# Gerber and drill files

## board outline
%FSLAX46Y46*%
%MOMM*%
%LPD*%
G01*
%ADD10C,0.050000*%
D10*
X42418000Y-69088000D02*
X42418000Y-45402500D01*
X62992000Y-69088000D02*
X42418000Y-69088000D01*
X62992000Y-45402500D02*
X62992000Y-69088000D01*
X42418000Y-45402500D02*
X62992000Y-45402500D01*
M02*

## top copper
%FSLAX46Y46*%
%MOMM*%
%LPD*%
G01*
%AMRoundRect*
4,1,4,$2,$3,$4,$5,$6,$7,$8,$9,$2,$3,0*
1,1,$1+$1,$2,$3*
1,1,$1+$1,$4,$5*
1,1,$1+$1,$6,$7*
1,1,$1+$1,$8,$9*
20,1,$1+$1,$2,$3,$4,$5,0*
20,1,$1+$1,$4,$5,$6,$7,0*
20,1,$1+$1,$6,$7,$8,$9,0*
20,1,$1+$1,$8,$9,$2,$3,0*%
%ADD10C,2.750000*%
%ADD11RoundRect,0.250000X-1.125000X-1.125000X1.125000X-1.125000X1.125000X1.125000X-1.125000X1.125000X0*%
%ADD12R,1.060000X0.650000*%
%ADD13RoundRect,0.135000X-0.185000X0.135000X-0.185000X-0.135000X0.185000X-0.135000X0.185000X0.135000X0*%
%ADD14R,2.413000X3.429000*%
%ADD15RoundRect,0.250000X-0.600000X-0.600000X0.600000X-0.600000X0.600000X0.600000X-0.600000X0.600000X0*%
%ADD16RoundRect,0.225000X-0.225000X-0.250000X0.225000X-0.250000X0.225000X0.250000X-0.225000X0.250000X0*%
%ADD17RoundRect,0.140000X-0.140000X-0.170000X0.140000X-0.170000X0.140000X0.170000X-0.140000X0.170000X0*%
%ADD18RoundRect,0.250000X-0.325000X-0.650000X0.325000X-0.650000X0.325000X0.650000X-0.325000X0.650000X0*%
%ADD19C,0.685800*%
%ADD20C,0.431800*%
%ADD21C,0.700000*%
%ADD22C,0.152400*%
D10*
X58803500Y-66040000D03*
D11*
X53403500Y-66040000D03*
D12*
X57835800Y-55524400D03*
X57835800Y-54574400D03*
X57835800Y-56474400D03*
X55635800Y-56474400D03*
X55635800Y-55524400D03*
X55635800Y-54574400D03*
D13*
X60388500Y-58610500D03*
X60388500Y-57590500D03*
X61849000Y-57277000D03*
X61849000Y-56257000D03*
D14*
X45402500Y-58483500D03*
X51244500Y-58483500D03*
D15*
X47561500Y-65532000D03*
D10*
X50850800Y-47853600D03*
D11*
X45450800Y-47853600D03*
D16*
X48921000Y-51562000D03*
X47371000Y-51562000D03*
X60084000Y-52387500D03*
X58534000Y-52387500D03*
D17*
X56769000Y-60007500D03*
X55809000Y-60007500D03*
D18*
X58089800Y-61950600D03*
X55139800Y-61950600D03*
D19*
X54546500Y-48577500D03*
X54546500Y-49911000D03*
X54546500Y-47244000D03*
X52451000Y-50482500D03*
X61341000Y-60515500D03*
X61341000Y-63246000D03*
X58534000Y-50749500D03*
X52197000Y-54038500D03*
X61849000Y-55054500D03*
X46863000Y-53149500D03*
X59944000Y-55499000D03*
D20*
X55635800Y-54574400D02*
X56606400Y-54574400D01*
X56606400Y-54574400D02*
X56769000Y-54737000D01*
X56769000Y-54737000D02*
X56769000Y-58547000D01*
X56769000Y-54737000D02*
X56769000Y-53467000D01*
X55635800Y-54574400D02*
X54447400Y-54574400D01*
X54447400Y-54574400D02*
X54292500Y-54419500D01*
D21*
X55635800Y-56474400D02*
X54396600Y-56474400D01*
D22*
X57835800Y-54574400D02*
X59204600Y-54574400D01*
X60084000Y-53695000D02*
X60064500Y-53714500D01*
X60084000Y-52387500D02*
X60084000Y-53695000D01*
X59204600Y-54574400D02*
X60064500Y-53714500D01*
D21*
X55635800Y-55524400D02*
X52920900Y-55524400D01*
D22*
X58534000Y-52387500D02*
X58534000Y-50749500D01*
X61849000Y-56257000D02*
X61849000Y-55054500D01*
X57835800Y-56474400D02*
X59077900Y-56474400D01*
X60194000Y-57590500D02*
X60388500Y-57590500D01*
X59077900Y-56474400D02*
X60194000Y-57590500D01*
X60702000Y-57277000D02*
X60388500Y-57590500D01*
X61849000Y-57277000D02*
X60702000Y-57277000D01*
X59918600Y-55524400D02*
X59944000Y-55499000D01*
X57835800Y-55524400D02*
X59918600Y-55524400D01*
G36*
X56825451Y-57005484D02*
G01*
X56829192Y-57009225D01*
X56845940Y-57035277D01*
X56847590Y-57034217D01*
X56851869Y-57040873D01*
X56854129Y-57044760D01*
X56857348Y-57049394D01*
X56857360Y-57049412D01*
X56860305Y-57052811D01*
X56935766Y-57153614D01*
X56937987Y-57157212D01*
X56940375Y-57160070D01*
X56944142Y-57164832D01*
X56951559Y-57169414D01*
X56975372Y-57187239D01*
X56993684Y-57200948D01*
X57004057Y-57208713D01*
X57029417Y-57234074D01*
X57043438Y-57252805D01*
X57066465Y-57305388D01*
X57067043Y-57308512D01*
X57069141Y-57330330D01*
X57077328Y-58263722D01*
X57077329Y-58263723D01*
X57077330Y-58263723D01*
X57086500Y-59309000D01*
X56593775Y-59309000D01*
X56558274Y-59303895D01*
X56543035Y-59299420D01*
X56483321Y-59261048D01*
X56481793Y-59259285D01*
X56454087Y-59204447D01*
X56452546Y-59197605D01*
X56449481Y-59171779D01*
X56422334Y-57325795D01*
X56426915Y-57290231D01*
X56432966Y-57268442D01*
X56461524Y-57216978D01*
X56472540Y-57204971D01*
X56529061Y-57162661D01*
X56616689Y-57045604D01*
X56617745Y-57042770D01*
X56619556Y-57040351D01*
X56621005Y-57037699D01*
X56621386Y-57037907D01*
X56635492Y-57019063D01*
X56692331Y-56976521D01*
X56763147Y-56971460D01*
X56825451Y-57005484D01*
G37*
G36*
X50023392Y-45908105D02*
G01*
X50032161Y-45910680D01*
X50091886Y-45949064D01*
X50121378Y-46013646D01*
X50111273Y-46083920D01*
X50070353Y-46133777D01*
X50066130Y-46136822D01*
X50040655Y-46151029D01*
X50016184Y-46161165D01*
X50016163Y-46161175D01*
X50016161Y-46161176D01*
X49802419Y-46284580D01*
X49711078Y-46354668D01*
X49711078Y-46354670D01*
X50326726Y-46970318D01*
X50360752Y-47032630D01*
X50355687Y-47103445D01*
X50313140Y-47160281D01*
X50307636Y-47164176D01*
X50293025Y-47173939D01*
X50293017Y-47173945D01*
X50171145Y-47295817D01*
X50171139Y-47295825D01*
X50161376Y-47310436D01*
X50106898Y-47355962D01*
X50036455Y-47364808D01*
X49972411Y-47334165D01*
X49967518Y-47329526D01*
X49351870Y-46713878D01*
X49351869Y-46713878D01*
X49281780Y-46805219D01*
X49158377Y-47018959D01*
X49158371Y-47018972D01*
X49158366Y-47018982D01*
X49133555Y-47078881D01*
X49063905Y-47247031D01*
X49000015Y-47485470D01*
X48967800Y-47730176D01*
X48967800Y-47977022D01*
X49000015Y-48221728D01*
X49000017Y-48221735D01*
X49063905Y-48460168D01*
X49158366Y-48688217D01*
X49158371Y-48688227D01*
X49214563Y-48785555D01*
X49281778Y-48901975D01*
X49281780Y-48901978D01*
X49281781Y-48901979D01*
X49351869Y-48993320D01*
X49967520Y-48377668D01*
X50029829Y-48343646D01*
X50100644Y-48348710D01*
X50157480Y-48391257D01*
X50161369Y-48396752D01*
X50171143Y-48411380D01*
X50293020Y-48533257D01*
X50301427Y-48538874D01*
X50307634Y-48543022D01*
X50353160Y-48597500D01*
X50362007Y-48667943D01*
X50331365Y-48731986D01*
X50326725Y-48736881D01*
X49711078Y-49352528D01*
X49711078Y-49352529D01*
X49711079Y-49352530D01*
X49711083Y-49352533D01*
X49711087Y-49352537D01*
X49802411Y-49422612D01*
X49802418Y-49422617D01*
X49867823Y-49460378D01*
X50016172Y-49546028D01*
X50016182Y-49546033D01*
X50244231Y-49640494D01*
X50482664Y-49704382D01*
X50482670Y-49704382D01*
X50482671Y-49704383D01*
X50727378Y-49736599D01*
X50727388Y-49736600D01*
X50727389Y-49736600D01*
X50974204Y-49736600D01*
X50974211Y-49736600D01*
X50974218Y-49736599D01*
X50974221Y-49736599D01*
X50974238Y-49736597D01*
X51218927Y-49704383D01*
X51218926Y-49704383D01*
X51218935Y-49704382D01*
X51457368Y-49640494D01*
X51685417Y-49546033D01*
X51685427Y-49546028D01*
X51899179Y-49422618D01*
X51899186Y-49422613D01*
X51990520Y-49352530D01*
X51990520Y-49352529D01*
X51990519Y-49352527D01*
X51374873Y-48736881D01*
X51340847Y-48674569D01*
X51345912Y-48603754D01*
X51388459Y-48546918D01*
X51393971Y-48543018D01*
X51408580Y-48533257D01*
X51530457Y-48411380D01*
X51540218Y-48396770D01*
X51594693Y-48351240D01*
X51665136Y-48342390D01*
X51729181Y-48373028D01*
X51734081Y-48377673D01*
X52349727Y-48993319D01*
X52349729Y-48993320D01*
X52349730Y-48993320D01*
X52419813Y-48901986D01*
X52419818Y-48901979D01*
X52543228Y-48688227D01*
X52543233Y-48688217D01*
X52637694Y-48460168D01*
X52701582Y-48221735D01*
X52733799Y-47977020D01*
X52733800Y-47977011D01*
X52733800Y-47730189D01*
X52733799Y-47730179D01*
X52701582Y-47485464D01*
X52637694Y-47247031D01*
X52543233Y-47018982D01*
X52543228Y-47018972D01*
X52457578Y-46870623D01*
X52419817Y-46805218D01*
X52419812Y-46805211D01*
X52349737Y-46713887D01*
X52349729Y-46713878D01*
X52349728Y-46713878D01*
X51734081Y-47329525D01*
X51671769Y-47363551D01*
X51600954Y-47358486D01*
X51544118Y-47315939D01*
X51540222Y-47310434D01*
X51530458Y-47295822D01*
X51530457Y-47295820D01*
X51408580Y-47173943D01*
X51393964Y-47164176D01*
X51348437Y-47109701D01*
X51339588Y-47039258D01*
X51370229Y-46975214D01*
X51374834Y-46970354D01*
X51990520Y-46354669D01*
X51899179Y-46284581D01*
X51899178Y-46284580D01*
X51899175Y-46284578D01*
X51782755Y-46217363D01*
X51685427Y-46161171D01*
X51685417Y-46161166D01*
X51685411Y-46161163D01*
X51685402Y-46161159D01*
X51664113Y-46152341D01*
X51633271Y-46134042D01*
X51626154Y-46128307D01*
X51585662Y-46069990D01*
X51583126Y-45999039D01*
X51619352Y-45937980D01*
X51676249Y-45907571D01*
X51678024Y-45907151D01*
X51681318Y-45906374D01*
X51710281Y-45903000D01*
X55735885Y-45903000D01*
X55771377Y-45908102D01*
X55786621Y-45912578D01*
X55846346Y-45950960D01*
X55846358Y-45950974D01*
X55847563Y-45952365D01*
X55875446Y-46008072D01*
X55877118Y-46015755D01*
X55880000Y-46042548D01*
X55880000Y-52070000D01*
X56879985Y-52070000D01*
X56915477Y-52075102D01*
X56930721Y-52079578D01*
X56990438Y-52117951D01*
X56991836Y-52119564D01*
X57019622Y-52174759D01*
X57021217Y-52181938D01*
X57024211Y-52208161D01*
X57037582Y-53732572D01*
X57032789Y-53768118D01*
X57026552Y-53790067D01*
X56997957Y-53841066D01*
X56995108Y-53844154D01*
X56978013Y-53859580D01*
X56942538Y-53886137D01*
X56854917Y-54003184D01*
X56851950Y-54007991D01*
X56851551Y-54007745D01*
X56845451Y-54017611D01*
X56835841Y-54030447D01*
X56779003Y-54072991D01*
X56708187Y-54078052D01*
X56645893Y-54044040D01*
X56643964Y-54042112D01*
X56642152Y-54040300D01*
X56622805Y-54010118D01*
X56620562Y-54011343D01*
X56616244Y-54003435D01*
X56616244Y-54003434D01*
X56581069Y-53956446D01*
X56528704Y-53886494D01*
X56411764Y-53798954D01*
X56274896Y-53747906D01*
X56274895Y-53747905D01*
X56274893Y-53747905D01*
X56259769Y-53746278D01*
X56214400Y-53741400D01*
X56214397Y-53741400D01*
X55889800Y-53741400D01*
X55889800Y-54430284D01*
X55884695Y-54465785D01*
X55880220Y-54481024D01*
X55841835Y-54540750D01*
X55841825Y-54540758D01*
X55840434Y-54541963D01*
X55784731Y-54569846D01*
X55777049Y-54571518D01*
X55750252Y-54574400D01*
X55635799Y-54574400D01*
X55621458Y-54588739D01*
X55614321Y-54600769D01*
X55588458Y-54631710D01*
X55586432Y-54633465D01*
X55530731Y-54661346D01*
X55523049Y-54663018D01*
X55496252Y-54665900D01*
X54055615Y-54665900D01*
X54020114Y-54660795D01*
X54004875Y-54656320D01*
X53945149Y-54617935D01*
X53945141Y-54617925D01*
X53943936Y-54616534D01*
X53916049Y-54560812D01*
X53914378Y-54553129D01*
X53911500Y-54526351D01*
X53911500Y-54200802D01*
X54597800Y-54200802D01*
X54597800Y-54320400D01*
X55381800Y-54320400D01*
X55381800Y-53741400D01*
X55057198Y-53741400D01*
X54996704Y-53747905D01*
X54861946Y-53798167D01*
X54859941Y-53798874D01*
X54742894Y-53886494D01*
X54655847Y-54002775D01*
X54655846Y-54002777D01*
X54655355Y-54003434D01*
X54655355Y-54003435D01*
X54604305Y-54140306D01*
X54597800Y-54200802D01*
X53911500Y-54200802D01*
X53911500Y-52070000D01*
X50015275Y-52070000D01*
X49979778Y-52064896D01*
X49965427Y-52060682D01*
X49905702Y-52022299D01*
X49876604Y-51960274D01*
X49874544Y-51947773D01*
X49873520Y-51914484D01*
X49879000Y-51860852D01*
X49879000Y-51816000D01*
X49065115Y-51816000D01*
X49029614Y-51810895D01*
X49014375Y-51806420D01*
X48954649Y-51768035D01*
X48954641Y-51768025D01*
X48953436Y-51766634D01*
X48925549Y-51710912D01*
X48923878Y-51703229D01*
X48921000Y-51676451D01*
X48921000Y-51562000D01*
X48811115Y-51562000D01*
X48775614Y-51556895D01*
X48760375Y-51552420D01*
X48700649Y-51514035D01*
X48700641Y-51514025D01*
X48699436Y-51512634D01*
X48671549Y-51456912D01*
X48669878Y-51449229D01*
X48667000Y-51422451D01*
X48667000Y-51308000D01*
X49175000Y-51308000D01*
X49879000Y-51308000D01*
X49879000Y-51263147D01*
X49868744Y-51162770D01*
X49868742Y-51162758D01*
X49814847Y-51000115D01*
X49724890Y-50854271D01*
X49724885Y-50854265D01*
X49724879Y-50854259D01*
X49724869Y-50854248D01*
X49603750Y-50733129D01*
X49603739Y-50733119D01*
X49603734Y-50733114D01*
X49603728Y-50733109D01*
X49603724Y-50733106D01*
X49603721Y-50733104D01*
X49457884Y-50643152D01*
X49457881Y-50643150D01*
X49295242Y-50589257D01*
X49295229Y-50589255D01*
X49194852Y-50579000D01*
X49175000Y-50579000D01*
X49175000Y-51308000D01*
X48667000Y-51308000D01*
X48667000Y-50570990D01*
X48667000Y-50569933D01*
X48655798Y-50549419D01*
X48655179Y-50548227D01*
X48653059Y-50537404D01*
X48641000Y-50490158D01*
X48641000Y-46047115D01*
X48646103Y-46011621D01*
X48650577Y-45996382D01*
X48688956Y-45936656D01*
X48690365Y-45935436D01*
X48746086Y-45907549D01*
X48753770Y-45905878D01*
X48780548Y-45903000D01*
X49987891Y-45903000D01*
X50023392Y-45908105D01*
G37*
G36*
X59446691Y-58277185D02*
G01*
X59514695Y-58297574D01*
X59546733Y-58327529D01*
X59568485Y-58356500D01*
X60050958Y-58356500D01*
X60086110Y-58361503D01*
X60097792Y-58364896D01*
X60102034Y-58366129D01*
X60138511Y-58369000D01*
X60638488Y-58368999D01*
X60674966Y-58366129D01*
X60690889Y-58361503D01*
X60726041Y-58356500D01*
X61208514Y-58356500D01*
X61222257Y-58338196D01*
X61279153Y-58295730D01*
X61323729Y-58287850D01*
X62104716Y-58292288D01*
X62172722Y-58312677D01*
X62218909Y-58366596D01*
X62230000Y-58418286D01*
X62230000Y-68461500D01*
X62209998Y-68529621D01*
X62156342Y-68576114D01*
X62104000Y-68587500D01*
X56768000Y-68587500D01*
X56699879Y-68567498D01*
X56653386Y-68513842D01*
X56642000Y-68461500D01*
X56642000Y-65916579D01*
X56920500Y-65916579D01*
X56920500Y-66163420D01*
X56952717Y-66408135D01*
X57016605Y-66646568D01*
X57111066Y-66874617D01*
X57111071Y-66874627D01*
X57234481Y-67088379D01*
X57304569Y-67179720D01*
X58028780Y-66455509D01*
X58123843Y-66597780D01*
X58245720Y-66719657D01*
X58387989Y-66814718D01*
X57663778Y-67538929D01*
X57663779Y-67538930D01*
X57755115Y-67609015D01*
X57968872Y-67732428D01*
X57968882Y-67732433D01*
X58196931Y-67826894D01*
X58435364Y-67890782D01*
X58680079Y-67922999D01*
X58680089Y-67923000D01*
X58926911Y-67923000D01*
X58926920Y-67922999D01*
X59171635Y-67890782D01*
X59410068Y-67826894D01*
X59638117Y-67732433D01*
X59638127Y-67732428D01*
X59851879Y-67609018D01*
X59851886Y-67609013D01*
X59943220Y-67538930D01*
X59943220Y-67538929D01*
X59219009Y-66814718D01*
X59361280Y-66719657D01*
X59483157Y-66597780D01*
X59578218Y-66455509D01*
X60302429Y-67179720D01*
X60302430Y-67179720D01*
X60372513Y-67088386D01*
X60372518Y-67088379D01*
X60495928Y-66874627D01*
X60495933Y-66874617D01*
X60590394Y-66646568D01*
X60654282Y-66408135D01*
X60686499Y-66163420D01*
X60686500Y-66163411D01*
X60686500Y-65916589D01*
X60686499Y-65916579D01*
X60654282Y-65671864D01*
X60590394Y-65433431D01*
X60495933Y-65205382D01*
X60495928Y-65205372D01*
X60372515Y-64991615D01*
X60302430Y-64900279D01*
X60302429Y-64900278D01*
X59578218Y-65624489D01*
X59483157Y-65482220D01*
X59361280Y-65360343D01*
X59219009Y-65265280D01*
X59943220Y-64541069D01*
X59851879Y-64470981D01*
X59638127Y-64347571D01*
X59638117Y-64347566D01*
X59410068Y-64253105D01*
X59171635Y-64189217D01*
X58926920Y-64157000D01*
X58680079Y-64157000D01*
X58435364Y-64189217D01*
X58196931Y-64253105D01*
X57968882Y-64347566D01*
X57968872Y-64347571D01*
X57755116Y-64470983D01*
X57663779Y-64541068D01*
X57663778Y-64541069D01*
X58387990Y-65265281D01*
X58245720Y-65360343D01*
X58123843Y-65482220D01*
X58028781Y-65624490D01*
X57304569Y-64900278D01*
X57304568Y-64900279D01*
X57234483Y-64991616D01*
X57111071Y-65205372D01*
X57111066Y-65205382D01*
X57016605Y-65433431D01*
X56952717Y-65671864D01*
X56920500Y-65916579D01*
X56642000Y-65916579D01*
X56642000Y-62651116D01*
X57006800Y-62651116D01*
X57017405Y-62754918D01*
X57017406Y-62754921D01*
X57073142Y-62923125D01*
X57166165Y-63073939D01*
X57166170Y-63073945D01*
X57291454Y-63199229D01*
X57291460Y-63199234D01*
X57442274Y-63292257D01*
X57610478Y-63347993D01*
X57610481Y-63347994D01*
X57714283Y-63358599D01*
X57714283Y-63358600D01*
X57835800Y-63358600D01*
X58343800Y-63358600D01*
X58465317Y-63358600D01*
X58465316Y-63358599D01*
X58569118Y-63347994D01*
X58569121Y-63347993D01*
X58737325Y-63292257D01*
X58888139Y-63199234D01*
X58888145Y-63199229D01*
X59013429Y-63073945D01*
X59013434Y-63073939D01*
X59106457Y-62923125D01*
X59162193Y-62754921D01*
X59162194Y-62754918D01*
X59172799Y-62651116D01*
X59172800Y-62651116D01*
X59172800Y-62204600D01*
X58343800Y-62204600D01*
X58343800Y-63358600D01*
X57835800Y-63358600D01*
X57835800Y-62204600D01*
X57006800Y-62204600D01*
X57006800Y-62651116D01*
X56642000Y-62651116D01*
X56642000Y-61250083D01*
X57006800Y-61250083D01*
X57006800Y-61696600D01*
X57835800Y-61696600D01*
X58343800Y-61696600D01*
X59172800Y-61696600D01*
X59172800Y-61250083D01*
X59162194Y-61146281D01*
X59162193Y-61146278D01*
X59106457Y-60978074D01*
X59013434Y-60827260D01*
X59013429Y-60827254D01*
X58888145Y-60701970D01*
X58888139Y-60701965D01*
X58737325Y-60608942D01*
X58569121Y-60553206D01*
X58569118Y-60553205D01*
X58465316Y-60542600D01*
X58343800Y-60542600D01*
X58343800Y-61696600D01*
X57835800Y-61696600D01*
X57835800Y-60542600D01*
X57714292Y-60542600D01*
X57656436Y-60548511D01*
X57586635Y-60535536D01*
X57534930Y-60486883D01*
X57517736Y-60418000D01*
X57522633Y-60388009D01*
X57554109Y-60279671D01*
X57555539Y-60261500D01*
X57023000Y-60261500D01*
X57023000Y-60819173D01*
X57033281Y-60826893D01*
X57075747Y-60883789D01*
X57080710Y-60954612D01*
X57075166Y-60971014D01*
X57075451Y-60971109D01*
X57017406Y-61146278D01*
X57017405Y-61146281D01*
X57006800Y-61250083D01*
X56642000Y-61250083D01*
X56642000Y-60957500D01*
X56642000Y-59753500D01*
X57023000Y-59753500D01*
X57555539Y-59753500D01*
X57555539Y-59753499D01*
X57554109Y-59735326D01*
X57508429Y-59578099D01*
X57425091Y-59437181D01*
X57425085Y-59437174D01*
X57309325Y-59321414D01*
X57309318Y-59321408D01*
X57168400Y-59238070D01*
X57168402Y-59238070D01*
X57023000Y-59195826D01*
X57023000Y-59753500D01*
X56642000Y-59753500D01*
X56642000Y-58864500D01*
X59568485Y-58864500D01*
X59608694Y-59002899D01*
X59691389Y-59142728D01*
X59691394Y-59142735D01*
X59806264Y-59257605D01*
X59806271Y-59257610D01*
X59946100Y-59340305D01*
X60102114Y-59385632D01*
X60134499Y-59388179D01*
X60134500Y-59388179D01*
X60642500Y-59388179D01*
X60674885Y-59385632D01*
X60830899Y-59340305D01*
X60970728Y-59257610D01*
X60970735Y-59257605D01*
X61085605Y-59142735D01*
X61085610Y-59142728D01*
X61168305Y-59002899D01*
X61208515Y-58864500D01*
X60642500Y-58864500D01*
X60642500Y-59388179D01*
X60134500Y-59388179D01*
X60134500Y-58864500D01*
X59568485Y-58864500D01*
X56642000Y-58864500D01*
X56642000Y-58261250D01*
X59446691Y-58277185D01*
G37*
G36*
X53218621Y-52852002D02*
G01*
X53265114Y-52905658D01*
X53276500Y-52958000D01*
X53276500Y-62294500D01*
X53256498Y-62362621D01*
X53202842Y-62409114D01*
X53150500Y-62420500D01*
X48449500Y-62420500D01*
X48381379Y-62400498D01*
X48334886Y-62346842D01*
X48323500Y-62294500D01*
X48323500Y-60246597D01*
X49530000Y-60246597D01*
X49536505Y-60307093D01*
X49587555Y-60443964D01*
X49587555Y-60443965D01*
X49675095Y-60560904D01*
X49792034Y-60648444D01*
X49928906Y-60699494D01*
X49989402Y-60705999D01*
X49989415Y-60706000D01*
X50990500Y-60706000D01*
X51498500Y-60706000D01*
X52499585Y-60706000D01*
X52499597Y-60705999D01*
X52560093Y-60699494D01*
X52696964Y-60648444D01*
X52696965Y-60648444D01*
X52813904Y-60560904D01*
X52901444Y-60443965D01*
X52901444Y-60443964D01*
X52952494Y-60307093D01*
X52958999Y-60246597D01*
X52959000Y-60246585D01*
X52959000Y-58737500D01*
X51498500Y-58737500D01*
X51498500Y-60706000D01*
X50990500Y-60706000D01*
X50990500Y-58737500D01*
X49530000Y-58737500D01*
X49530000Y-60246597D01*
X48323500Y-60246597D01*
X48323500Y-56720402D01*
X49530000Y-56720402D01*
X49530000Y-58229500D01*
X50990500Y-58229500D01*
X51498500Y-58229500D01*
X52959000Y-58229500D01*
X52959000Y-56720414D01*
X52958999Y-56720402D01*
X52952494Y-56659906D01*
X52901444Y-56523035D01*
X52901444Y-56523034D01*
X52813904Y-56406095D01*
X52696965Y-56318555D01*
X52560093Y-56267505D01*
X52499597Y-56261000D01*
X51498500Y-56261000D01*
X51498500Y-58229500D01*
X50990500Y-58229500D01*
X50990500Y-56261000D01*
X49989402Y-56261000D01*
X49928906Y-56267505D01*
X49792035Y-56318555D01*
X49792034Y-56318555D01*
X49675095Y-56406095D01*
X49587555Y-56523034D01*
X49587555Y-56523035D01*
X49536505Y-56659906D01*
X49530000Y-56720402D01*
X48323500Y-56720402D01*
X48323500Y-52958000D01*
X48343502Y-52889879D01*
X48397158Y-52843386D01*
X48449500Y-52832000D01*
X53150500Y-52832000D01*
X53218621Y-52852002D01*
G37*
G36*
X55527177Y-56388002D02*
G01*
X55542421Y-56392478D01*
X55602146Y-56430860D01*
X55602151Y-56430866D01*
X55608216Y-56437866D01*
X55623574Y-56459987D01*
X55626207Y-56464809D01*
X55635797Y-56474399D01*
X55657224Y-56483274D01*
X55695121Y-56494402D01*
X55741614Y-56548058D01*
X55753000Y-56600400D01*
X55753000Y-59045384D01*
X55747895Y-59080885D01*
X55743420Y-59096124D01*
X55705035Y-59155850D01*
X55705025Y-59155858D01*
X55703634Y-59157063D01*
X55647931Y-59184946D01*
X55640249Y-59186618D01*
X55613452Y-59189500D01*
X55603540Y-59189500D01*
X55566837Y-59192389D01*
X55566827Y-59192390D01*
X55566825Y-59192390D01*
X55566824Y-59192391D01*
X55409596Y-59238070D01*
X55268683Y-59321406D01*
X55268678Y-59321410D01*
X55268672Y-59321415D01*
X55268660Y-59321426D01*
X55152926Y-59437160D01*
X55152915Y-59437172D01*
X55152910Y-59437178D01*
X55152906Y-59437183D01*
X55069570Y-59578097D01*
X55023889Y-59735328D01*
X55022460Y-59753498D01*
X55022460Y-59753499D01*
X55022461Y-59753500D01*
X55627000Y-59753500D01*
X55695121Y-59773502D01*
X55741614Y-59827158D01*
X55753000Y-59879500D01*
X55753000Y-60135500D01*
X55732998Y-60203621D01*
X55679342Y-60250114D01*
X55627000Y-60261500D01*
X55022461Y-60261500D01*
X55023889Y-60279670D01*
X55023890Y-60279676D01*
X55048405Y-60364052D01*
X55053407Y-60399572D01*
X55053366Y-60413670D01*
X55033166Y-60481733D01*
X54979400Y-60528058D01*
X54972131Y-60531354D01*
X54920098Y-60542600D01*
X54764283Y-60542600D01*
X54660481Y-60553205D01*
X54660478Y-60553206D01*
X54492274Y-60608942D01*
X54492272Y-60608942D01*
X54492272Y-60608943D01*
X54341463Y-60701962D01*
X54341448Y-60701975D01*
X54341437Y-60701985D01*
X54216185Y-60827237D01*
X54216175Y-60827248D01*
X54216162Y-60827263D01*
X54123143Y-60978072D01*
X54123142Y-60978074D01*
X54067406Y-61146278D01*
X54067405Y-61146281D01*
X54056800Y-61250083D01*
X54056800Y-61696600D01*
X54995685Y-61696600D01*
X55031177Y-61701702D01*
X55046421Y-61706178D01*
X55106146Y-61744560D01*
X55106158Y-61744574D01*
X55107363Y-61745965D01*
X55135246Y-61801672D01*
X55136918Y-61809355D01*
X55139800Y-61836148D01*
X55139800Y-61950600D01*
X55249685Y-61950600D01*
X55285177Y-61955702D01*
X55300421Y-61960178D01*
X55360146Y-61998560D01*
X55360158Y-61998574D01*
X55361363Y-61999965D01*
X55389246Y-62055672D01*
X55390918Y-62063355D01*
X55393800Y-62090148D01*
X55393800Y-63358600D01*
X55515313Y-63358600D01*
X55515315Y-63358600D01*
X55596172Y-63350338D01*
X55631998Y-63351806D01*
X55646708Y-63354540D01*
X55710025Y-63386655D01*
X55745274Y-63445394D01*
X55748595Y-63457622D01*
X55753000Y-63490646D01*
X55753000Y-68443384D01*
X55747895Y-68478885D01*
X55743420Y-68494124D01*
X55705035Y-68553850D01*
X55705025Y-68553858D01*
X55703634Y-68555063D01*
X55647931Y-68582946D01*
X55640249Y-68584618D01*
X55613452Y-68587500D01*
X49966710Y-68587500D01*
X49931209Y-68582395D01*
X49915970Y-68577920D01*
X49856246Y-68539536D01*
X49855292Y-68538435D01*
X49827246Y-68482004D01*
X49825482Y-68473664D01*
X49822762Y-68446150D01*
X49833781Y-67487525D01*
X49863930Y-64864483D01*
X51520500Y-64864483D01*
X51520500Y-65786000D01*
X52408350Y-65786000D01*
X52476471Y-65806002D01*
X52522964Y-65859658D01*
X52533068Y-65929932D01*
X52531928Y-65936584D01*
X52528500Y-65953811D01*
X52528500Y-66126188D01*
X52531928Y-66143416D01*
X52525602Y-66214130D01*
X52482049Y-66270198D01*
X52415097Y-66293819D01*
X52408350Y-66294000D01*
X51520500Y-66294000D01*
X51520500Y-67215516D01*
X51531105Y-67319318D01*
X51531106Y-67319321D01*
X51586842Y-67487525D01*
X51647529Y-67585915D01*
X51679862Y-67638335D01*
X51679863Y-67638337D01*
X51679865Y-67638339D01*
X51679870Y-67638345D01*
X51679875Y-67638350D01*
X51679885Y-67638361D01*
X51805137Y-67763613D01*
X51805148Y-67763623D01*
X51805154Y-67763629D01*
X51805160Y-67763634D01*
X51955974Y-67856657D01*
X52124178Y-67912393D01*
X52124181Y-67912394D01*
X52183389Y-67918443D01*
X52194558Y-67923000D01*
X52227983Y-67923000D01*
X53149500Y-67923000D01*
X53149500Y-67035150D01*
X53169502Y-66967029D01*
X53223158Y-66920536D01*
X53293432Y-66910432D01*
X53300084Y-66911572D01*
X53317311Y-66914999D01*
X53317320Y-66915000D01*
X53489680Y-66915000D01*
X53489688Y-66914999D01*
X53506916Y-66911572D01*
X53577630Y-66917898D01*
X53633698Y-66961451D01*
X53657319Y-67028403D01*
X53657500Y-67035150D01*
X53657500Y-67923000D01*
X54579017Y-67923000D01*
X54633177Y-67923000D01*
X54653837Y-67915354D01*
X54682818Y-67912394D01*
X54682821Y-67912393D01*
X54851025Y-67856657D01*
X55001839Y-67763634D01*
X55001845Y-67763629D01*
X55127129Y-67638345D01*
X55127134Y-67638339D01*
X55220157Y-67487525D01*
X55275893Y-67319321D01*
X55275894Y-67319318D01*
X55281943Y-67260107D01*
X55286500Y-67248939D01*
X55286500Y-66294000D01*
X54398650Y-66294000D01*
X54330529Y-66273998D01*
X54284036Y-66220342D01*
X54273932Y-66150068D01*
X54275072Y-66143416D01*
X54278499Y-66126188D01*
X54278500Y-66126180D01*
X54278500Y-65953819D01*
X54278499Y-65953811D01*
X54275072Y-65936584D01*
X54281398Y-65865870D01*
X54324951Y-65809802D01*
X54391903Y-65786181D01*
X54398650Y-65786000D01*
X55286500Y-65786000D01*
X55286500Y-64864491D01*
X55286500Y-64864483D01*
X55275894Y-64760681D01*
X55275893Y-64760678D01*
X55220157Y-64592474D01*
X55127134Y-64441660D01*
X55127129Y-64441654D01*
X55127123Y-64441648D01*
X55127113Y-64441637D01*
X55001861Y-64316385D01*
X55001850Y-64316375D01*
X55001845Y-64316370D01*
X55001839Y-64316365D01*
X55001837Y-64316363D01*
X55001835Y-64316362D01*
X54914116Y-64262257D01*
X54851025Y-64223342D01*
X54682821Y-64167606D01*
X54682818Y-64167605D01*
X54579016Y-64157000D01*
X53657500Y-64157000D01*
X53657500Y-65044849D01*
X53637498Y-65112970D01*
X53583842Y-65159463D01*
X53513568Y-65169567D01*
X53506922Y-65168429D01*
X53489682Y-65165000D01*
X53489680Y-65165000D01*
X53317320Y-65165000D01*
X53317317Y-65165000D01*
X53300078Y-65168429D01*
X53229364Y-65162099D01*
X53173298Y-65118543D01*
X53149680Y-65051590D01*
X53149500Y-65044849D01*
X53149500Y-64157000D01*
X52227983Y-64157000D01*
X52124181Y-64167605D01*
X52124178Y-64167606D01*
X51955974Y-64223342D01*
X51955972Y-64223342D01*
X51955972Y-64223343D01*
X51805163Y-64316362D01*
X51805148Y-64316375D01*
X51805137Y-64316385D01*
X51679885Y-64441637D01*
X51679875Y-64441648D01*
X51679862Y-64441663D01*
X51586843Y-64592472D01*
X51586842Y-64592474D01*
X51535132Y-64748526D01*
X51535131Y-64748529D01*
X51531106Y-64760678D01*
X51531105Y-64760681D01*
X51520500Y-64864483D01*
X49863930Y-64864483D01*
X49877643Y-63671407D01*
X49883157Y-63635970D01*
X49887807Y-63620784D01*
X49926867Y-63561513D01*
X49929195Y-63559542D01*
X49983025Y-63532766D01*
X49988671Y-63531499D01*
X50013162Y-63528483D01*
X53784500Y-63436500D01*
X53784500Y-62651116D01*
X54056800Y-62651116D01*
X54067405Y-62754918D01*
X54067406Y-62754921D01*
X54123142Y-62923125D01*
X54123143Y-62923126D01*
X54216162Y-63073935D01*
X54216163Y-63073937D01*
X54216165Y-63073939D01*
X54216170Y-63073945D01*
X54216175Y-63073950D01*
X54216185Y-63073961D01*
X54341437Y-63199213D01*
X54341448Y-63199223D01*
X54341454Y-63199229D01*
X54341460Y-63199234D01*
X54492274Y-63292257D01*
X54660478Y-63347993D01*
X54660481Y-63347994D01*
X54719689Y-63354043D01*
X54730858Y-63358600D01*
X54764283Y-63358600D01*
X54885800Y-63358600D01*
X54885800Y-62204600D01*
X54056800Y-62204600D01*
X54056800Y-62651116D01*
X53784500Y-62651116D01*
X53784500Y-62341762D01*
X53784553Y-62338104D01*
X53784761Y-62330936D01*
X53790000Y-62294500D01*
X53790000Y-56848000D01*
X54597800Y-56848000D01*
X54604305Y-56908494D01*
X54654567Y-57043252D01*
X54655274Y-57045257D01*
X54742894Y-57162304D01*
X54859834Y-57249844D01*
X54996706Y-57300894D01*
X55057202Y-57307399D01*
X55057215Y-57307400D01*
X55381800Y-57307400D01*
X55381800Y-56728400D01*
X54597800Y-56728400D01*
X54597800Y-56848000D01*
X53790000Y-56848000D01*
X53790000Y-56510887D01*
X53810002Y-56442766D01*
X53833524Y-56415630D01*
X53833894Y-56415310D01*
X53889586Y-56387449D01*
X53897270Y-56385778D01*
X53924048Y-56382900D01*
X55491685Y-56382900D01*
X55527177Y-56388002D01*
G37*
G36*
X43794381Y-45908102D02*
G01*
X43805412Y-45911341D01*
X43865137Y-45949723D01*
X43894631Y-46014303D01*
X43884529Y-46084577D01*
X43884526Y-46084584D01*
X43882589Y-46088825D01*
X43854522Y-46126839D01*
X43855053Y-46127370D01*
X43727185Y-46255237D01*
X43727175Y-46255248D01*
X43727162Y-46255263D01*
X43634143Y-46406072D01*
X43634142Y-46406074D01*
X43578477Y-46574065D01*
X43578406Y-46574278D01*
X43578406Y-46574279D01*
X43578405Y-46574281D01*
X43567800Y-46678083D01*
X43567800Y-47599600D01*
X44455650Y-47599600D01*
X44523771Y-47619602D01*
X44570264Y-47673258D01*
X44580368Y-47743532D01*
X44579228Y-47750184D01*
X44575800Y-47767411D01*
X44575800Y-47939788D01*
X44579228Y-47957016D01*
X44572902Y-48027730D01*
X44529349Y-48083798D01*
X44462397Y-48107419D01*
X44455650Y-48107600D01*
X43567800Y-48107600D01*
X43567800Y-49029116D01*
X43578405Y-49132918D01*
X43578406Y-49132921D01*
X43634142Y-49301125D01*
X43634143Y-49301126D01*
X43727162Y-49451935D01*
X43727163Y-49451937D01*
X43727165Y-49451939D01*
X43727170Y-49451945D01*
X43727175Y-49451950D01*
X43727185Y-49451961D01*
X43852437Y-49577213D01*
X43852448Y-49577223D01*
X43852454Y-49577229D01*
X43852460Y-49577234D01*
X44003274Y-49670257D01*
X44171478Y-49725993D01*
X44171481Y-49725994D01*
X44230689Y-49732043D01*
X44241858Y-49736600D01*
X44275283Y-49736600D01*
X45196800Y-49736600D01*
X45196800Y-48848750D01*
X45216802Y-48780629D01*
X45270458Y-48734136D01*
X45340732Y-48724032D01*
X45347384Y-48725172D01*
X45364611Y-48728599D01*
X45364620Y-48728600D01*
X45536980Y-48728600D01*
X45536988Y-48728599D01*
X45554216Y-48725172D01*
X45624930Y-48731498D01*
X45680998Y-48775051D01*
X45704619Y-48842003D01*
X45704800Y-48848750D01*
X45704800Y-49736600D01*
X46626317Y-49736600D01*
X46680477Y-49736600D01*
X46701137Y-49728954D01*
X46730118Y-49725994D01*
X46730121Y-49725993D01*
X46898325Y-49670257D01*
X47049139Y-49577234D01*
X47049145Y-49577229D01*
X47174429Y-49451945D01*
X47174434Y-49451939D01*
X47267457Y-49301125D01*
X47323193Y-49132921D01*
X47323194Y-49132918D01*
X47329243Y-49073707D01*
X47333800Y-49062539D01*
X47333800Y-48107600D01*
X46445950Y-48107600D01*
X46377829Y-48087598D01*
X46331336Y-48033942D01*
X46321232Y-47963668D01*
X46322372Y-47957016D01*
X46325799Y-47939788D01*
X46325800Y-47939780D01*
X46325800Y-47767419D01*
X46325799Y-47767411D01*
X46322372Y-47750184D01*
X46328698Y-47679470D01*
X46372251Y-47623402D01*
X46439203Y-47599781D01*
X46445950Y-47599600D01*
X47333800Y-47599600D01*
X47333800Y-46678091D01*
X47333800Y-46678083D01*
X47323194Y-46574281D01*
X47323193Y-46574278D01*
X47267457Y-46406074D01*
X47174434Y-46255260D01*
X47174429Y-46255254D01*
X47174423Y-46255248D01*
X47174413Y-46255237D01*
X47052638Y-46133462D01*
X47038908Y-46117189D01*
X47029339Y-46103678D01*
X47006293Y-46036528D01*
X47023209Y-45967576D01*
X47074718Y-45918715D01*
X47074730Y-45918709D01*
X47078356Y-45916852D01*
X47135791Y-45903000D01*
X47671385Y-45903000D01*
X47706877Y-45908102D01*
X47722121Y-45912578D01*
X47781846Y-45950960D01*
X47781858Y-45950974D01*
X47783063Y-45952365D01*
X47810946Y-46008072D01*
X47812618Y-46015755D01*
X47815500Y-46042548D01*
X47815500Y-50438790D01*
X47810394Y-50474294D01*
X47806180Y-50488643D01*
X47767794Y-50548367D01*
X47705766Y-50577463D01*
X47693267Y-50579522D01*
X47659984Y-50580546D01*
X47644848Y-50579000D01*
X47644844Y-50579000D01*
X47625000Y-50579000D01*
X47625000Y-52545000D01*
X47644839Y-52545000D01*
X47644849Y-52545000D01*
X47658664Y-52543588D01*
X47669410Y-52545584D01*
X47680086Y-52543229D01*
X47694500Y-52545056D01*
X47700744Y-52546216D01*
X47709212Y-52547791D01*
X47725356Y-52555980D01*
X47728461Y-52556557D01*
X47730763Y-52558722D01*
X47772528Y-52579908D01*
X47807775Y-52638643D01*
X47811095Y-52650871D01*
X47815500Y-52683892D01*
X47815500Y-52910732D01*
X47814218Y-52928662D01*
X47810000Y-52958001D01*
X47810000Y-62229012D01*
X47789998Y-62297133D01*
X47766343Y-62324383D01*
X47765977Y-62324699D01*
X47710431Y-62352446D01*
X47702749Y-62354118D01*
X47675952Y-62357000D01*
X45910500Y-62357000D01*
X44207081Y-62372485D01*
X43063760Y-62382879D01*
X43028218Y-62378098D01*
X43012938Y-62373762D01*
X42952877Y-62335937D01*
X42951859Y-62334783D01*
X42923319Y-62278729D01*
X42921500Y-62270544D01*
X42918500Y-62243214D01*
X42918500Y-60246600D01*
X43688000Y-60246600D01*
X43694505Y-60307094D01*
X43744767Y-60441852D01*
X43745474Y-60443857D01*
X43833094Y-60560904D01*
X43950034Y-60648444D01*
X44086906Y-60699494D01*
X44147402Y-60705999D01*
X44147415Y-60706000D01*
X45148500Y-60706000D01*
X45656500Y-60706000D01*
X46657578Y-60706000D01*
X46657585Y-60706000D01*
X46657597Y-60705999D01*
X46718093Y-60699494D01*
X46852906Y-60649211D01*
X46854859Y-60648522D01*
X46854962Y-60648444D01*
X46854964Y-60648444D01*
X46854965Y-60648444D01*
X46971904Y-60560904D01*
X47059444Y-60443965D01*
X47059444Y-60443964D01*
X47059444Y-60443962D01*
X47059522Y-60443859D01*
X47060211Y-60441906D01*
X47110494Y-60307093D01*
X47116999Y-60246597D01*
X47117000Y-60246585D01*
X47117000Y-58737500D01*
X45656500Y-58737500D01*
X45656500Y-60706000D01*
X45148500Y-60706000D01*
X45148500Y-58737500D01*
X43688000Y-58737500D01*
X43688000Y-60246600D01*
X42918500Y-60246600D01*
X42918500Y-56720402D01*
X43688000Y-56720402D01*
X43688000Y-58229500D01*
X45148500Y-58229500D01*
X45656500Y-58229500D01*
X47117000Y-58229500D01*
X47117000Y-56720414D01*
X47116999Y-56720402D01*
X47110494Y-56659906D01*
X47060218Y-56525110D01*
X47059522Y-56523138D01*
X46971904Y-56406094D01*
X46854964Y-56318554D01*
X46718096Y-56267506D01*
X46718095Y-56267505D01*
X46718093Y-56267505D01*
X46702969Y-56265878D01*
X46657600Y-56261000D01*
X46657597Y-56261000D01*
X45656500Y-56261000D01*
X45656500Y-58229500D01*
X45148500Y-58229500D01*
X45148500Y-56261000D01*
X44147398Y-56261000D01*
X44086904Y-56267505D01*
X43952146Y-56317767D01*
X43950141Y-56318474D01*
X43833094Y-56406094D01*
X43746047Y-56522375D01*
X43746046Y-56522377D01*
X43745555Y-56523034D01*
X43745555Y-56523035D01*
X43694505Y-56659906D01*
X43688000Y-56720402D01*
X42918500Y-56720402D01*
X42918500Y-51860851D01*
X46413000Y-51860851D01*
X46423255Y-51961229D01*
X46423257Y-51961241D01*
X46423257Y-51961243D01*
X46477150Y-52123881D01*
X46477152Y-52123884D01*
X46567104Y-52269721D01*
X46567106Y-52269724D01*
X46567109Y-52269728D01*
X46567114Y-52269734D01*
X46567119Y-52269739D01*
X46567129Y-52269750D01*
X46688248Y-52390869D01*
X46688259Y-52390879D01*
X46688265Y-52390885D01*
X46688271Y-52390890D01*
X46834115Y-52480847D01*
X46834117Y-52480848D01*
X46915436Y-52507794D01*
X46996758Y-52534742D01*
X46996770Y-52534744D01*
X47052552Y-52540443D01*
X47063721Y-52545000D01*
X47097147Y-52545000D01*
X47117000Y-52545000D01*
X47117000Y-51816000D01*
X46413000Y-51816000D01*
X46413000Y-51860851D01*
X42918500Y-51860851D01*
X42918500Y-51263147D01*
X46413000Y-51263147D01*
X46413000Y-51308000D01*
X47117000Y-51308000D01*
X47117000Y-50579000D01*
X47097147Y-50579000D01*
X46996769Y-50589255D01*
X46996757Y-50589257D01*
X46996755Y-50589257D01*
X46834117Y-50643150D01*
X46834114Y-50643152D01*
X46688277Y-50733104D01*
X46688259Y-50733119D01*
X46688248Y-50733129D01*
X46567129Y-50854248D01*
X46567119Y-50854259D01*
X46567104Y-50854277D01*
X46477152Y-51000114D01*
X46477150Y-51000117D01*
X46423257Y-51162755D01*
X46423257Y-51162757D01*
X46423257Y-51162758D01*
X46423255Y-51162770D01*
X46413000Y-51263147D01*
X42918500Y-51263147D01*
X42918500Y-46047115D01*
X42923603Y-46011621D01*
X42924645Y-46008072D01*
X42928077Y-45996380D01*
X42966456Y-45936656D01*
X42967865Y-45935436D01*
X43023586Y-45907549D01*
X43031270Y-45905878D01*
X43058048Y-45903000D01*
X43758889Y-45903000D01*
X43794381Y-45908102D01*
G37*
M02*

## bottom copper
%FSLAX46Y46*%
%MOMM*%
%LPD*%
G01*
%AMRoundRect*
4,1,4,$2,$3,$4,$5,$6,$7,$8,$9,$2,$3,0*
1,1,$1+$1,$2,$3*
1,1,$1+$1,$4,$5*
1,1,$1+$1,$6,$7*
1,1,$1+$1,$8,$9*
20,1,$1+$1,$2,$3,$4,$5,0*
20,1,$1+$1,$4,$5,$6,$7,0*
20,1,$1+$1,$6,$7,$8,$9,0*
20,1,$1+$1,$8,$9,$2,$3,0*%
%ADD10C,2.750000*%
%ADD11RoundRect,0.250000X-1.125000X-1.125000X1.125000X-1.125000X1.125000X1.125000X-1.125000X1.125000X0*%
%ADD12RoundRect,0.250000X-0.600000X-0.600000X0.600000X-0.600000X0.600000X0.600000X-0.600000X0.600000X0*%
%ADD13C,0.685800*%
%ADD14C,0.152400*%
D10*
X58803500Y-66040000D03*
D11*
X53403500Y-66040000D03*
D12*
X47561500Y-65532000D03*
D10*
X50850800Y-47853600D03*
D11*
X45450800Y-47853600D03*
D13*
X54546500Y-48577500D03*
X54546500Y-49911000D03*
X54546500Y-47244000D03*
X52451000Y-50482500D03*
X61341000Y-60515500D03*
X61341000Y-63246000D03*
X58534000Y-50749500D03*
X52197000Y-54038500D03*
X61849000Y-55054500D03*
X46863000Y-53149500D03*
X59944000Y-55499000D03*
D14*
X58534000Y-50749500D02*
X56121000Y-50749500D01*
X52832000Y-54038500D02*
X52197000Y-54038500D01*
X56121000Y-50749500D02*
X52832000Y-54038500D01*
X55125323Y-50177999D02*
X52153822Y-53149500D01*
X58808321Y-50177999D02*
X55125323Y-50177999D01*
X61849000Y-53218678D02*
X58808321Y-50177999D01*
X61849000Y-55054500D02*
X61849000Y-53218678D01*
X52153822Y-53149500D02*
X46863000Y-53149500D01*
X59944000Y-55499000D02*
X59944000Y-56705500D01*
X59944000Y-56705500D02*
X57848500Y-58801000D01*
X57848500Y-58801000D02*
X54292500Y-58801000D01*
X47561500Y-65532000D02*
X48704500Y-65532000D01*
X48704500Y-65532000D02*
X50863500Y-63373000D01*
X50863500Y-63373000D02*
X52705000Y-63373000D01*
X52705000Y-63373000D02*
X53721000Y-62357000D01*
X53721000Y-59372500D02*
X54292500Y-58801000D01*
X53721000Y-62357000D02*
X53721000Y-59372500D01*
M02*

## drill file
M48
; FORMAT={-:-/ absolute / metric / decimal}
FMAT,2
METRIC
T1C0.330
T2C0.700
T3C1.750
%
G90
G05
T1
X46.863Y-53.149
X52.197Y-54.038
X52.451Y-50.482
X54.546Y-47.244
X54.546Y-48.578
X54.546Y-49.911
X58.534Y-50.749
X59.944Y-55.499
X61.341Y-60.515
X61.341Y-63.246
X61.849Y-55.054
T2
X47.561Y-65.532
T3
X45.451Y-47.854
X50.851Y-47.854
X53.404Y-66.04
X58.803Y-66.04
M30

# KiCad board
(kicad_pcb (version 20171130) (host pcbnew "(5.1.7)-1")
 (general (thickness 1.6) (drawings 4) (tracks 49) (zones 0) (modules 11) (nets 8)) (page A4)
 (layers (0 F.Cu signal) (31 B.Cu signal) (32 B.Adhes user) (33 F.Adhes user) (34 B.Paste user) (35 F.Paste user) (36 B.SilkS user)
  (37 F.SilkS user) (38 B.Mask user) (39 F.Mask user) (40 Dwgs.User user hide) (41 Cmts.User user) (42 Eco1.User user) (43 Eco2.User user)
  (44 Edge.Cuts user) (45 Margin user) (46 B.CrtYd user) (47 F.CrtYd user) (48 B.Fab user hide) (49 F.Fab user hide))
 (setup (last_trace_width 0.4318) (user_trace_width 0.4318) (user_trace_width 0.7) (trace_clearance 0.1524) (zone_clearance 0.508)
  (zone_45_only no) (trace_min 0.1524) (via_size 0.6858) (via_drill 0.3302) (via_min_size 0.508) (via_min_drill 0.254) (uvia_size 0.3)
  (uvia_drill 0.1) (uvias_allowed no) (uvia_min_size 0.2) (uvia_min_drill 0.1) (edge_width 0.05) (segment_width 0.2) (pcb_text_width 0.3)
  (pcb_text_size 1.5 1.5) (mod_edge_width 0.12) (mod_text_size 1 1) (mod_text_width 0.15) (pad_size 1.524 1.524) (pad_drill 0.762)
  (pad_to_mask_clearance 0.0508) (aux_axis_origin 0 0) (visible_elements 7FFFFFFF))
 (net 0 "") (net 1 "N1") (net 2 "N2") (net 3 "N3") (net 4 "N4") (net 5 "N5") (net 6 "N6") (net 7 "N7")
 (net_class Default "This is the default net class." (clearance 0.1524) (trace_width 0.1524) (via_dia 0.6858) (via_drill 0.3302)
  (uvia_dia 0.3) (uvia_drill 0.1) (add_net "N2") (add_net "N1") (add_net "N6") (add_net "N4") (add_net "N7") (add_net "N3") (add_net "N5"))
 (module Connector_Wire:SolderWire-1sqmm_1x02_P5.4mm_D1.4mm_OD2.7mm (layer F.Cu) (at 53.4035 66.04)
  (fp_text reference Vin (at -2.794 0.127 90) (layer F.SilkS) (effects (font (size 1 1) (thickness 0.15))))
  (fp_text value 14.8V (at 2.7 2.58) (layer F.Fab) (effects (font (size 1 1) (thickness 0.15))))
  (pad 2 thru_hole circle (at 5.4 0) (size 2.75 2.75) (drill 1.75) (layers *.Cu *.Mask) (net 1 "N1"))
  (pad 1 thru_hole roundrect (at 0 0) (size 2.75 2.75) (drill 1.75) (layers *.Cu *.Mask) (roundrect_rratio 0.090909) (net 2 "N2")))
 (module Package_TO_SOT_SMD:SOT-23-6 (layer F.Cu) (at 56.7358 55.5244)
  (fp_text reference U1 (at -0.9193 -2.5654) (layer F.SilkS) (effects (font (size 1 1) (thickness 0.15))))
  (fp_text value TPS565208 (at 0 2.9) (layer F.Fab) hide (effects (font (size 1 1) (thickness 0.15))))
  (pad 5 smd rect (at 1.1 0) (size 1.06 0.65) (layers F.Cu F.Paste F.Mask) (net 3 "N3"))
  (pad 6 smd rect (at 1.1 -0.95) (size 1.06 0.65) (layers F.Cu F.Paste F.Mask) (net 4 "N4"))
  (pad 4 smd rect (at 1.1 0.95) (size 1.06 0.65) (layers F.Cu F.Paste F.Mask) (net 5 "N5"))
  (pad 3 smd rect (at -1.1 0.95) (size 1.06 0.65) (layers F.Cu F.Paste F.Mask) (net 2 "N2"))
  (pad 2 smd rect (at -1.1 0) (size 1.06 0.65) (layers F.Cu F.Paste F.Mask) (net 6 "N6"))
  (pad 1 smd rect (at -1.1 -0.95) (size 1.06 0.65) (layers F.Cu F.Paste F.Mask) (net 1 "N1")))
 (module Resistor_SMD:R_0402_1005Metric (layer F.Cu) (at 60.3885 58.1005 270)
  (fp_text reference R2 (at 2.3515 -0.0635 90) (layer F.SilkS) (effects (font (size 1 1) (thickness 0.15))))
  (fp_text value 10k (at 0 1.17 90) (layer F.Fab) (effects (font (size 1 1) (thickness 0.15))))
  (pad 2 smd roundrect (at 0.51 0 270) (size 0.54 0.64) (layers F.Cu F.Paste F.Mask) (roundrect_rratio 0.25) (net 1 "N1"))
  (pad 1 smd roundrect (at -0.51 0 270) (size 0.54 0.64) (layers F.Cu F.Paste F.Mask) (roundrect_rratio 0.25) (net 5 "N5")))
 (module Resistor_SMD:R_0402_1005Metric (layer F.Cu) (at 61.849 56.767 270)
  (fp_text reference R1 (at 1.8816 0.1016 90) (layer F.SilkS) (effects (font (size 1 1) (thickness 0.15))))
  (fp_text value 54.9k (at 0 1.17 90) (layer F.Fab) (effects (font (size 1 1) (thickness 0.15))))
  (pad 2 smd roundrect (at 0.51 0 270) (size 0.54 0.64) (layers F.Cu F.Paste F.Mask) (roundrect_rratio 0.25) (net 5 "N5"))
  (pad 1 smd roundrect (at -0.51 0 270) (size 0.54 0.64) (layers F.Cu F.Paste F.Mask) (roundrect_rratio 0.25) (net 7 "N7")))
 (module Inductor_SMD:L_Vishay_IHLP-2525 (layer F.Cu) (at 48.3235 58.4835 180)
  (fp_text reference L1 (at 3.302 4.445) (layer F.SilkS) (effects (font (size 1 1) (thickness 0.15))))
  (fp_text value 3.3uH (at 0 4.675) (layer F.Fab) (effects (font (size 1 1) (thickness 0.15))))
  (pad 2 smd rect (at 2.921 0 180) (size 2.413 3.429) (layers F.Cu F.Paste F.Mask) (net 7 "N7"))
  (pad 1 smd rect (at -2.921 0 180) (size 2.413 3.429) (layers F.Cu F.Paste F.Mask) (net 6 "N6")))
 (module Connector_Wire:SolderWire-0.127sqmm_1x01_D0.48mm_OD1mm (layer F.Cu) (at 47.5615 65.532)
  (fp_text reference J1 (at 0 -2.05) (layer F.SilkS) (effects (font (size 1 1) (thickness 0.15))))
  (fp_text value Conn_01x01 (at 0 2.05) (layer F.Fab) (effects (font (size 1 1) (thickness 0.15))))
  (pad 1 thru_hole roundrect (at 0 0) (size 1.7 1.7) (drill 0.7) (layers *.Cu *.Mask) (roundrect_rratio 0.147059) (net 3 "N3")))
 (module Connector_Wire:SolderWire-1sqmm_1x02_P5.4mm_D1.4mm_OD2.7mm (layer F.Cu) (at 45.4508 47.8536)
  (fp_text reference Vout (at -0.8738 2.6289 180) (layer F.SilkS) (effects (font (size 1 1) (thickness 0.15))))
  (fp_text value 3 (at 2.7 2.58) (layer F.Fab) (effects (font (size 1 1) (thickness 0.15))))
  (pad 2 thru_hole circle (at 5.4 0) (size 2.75 2.75) (drill 1.75) (layers *.Cu *.Mask) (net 1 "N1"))
  (pad 1 thru_hole roundrect (at 0 0) (size 2.75 2.75) (drill 1.75) (layers *.Cu *.Mask) (roundrect_rratio 0.090909) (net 7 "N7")))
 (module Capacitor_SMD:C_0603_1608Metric (layer F.Cu) (at 48.146 51.562)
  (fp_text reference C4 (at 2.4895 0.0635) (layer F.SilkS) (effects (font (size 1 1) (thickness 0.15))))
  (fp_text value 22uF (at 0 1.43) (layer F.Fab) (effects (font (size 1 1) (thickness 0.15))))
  (pad 2 smd roundrect (at 0.775 0) (size 0.9 0.95) (layers F.Cu F.Paste F.Mask) (roundrect_rratio 0.25) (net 1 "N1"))
  (pad 1 smd roundrect (at -0.775 0) (size 0.9 0.95) (layers F.Cu F.Paste F.Mask) (roundrect_rratio 0.25) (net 7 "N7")))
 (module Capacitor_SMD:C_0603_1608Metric (layer F.Cu) (at 59.309 52.3875)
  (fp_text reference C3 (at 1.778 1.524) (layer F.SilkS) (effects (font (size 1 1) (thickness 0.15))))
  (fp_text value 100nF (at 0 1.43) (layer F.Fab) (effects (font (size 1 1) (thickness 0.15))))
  (pad 2 smd roundrect (at 0.775 0) (size 0.9 0.95) (layers F.Cu F.Paste F.Mask) (roundrect_rratio 0.25) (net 4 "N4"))
  (pad 1 smd roundrect (at -0.775 0) (size 0.9 0.95) (layers F.Cu F.Paste F.Mask) (roundrect_rratio 0.25) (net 6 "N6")))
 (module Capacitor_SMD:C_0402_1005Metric (layer F.Cu) (at 56.289 60.0075)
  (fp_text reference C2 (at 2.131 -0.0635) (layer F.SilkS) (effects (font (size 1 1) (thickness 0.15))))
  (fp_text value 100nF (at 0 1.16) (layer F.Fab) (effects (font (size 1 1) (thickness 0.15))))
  (pad 2 smd roundrect (at 0.48 0) (size 0.56 0.62) (layers F.Cu F.Paste F.Mask) (roundrect_rratio 0.25) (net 1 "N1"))
  (pad 1 smd roundrect (at -0.48 0) (size 0.56 0.62) (layers F.Cu F.Paste F.Mask) (roundrect_rratio 0.25) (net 2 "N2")))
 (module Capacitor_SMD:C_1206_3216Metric (layer F.Cu) (at 56.6148 61.9506)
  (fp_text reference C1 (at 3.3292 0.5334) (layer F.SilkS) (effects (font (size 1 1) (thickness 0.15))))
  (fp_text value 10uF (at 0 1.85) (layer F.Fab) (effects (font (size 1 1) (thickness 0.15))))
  (pad 2 smd roundrect (at 1.475 0) (size 1.15 1.8) (layers F.Cu F.Paste F.Mask) (roundrect_rratio 0.217391) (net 1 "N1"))
  (pad 1 smd roundrect (at -1.475 0) (size 1.15 1.8) (layers F.Cu F.Paste F.Mask) (roundrect_rratio 0.217391) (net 2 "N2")))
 (gr_line (start 42.418 69.088) (end 42.418 45.4025) (layer Edge.Cuts) (width 0.05))
 (gr_line (start 62.992 69.088) (end 42.418 69.088) (layer Edge.Cuts) (width 0.05))
 (gr_line (start 62.992 45.4025) (end 62.992 69.088) (layer Edge.Cuts) (width 0.05))
 (gr_line (start 42.418 45.4025) (end 62.992 45.4025) (layer Edge.Cuts) (width 0.05))
 (via (at 54.5465 48.5775) (size 0.6858) (drill 0.3302) (layers F.Cu B.Cu) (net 1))
 (via (at 54.5465 49.911) (size 0.6858) (drill 0.3302) (layers F.Cu B.Cu) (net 1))
 (via (at 54.5465 47.244) (size 0.6858) (drill 0.3302) (layers F.Cu B.Cu) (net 1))
 (via (at 52.451 50.4825) (size 0.6858) (drill 0.3302) (layers F.Cu B.Cu) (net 1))
 (via (at 61.341 60.5155) (size 0.6858) (drill 0.3302) (layers F.Cu B.Cu) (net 1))
 (via (at 61.341 63.246) (size 0.6858) (drill 0.3302) (layers F.Cu B.Cu) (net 1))
 (segment (start 55.6358 54.5744) (end 56.6064 54.5744) (width 0.4318) (layer F.Cu) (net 1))
 (segment (start 56.6064 54.5744) (end 56.769 54.737) (width 0.4318) (layer F.Cu) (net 1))
 (segment (start 56.769 54.737) (end 56.769 58.547) (width 0.4318) (layer F.Cu) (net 1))
 (segment (start 56.769 54.737) (end 56.769 53.467) (width 0.4318) (layer F.Cu) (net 1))
 (segment (start 55.6358 54.5744) (end 54.4474 54.5744) (width 0.4318) (layer F.Cu) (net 1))
 (segment (start 54.4474 54.5744) (end 54.2925 54.4195) (width 0.4318) (layer F.Cu) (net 1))
 (segment (start 55.6358 56.4744) (end 54.3966 56.4744) (width 0.7) (layer F.Cu) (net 2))
 (segment (start 57.8358 54.5744) (end 59.2046 54.5744) (width 0.1524) (layer F.Cu) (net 4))
 (segment (start 60.084 53.695) (end 60.0645 53.7145) (width 0.1524) (layer F.Cu) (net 4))
 (segment (start 60.084 52.3875) (end 60.084 53.695) (width 0.1524) (layer F.Cu) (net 4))
 (segment (start 59.2046 54.5744) (end 60.0645 53.7145) (width 0.1524) (layer F.Cu) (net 4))
 (segment (start 55.6358 55.5244) (end 52.9209 55.5244) (width 0.7) (layer F.Cu) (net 6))
 (segment (start 58.534 52.3875) (end 58.534 50.7495) (width 0.1524) (layer F.Cu) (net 6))
 (via (at 58.534 50.7495) (size 0.6858) (drill 0.3302) (layers F.Cu B.Cu) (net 6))
 (segment (start 58.534 50.7495) (end 56.121 50.7495) (width 0.1524) (layer B.Cu) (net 6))
 (via (at 52.197 54.0385) (size 0.6858) (drill 0.3302) (layers F.Cu B.Cu) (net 6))
 (segment (start 52.832 54.0385) (end 52.197 54.0385) (width 0.1524) (layer B.Cu) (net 6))
 (segment (start 56.121 50.7495) (end 52.832 54.0385) (width 0.1524) (layer B.Cu) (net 6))
 (via (at 61.849 55.0545) (size 0.6858) (drill 0.3302) (layers F.Cu B.Cu) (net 7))
 (segment (start 61.849 56.257) (end 61.849 55.0545) (width 0.1524) (layer F.Cu) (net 7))
 (segment (start 55.125323 50.177999) (end 52.153822 53.1495) (width 0.1524) (layer B.Cu) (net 7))
 (segment (start 58.808321 50.177999) (end 55.125323 50.177999) (width 0.1524) (layer B.Cu) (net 7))
 (segment (start 61.849 53.218678) (end 58.808321 50.177999) (width 0.1524) (layer B.Cu) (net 7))
 (segment (start 61.849 55.0545) (end 61.849 53.218678) (width 0.1524) (layer B.Cu) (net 7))
 (via (at 46.863 53.1495) (size 0.6858) (drill 0.3302) (layers F.Cu B.Cu) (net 7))
 (segment (start 52.153822 53.1495) (end 46.863 53.1495) (width 0.1524) (layer B.Cu) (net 7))
 (segment (start 57.8358 56.4744) (end 59.0779 56.4744) (width 0.1524) (layer F.Cu) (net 5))
 (segment (start 60.194 57.5905) (end 60.3885 57.5905) (width 0.1524) (layer F.Cu) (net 5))
 (segment (start 59.0779 56.4744) (end 60.194 57.5905) (width 0.1524) (layer F.Cu) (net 5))
 (segment (start 60.702 57.277) (end 60.3885 57.5905) (width 0.1524) (layer F.Cu) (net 5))
 (segment (start 61.849 57.277) (end 60.702 57.277) (width 0.1524) (layer F.Cu) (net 5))
 (via (at 59.944 55.499) (size 0.6858) (drill 0.3302) (layers F.Cu B.Cu) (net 3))
 (segment (start 59.9186 55.5244) (end 59.944 55.499) (width 0.1524) (layer F.Cu) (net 3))
 (segment (start 57.8358 55.5244) (end 59.9186 55.5244) (width 0.1524) (layer F.Cu) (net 3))
 (segment (start 59.944 55.499) (end 59.944 56.7055) (width 0.1524) (layer B.Cu) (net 3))
 (segment (start 59.944 56.7055) (end 57.8485 58.801) (width 0.1524) (layer B.Cu) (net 3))
 (segment (start 57.8485 58.801) (end 54.2925 58.801) (width 0.1524) (layer B.Cu) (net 3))
 (segment (start 47.5615 65.532) (end 48.7045 65.532) (width 0.1524) (layer B.Cu) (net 3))
 (segment (start 48.7045 65.532) (end 50.8635 63.373) (width 0.1524) (layer B.Cu) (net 3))
 (segment (start 50.8635 63.373) (end 52.705 63.373) (width 0.1524) (layer B.Cu) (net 3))
 (segment (start 52.705 63.373) (end 53.721 62.357) (width 0.1524) (layer B.Cu) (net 3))
 (segment (start 53.721 59.3725) (end 54.2925 58.801) (width 0.1524) (layer B.Cu) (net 3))
 (segment (start 53.721 62.357) (end 53.721 59.3725) (width 0.1524) (layer B.Cu) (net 3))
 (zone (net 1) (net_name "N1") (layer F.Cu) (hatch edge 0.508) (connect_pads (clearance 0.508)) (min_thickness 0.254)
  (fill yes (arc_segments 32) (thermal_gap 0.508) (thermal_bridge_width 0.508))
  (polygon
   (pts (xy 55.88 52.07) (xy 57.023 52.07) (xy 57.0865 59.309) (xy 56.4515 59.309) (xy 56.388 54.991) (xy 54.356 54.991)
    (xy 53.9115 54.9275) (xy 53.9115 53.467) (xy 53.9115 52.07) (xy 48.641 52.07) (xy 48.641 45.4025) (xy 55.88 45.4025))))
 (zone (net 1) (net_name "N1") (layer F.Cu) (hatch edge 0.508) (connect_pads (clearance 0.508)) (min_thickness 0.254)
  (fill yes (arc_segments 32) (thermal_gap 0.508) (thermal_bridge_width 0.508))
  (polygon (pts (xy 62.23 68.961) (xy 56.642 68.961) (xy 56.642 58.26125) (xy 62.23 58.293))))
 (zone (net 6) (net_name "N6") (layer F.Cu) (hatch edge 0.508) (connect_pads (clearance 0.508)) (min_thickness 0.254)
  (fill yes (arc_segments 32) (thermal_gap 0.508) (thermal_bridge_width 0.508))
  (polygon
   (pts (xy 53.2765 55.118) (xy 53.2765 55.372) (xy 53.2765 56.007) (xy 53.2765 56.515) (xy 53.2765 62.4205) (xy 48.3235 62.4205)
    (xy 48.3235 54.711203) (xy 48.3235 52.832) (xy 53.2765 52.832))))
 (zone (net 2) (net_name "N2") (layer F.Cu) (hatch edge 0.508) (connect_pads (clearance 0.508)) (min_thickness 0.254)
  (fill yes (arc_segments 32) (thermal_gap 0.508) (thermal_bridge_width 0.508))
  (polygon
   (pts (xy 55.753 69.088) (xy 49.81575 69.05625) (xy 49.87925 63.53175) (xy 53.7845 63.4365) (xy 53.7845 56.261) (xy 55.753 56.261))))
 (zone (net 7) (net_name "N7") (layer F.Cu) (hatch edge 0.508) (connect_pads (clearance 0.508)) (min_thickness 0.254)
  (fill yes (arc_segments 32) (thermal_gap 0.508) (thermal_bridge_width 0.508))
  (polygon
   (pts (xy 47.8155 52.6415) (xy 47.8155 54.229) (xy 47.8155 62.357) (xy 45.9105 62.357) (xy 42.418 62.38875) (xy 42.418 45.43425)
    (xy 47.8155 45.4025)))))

